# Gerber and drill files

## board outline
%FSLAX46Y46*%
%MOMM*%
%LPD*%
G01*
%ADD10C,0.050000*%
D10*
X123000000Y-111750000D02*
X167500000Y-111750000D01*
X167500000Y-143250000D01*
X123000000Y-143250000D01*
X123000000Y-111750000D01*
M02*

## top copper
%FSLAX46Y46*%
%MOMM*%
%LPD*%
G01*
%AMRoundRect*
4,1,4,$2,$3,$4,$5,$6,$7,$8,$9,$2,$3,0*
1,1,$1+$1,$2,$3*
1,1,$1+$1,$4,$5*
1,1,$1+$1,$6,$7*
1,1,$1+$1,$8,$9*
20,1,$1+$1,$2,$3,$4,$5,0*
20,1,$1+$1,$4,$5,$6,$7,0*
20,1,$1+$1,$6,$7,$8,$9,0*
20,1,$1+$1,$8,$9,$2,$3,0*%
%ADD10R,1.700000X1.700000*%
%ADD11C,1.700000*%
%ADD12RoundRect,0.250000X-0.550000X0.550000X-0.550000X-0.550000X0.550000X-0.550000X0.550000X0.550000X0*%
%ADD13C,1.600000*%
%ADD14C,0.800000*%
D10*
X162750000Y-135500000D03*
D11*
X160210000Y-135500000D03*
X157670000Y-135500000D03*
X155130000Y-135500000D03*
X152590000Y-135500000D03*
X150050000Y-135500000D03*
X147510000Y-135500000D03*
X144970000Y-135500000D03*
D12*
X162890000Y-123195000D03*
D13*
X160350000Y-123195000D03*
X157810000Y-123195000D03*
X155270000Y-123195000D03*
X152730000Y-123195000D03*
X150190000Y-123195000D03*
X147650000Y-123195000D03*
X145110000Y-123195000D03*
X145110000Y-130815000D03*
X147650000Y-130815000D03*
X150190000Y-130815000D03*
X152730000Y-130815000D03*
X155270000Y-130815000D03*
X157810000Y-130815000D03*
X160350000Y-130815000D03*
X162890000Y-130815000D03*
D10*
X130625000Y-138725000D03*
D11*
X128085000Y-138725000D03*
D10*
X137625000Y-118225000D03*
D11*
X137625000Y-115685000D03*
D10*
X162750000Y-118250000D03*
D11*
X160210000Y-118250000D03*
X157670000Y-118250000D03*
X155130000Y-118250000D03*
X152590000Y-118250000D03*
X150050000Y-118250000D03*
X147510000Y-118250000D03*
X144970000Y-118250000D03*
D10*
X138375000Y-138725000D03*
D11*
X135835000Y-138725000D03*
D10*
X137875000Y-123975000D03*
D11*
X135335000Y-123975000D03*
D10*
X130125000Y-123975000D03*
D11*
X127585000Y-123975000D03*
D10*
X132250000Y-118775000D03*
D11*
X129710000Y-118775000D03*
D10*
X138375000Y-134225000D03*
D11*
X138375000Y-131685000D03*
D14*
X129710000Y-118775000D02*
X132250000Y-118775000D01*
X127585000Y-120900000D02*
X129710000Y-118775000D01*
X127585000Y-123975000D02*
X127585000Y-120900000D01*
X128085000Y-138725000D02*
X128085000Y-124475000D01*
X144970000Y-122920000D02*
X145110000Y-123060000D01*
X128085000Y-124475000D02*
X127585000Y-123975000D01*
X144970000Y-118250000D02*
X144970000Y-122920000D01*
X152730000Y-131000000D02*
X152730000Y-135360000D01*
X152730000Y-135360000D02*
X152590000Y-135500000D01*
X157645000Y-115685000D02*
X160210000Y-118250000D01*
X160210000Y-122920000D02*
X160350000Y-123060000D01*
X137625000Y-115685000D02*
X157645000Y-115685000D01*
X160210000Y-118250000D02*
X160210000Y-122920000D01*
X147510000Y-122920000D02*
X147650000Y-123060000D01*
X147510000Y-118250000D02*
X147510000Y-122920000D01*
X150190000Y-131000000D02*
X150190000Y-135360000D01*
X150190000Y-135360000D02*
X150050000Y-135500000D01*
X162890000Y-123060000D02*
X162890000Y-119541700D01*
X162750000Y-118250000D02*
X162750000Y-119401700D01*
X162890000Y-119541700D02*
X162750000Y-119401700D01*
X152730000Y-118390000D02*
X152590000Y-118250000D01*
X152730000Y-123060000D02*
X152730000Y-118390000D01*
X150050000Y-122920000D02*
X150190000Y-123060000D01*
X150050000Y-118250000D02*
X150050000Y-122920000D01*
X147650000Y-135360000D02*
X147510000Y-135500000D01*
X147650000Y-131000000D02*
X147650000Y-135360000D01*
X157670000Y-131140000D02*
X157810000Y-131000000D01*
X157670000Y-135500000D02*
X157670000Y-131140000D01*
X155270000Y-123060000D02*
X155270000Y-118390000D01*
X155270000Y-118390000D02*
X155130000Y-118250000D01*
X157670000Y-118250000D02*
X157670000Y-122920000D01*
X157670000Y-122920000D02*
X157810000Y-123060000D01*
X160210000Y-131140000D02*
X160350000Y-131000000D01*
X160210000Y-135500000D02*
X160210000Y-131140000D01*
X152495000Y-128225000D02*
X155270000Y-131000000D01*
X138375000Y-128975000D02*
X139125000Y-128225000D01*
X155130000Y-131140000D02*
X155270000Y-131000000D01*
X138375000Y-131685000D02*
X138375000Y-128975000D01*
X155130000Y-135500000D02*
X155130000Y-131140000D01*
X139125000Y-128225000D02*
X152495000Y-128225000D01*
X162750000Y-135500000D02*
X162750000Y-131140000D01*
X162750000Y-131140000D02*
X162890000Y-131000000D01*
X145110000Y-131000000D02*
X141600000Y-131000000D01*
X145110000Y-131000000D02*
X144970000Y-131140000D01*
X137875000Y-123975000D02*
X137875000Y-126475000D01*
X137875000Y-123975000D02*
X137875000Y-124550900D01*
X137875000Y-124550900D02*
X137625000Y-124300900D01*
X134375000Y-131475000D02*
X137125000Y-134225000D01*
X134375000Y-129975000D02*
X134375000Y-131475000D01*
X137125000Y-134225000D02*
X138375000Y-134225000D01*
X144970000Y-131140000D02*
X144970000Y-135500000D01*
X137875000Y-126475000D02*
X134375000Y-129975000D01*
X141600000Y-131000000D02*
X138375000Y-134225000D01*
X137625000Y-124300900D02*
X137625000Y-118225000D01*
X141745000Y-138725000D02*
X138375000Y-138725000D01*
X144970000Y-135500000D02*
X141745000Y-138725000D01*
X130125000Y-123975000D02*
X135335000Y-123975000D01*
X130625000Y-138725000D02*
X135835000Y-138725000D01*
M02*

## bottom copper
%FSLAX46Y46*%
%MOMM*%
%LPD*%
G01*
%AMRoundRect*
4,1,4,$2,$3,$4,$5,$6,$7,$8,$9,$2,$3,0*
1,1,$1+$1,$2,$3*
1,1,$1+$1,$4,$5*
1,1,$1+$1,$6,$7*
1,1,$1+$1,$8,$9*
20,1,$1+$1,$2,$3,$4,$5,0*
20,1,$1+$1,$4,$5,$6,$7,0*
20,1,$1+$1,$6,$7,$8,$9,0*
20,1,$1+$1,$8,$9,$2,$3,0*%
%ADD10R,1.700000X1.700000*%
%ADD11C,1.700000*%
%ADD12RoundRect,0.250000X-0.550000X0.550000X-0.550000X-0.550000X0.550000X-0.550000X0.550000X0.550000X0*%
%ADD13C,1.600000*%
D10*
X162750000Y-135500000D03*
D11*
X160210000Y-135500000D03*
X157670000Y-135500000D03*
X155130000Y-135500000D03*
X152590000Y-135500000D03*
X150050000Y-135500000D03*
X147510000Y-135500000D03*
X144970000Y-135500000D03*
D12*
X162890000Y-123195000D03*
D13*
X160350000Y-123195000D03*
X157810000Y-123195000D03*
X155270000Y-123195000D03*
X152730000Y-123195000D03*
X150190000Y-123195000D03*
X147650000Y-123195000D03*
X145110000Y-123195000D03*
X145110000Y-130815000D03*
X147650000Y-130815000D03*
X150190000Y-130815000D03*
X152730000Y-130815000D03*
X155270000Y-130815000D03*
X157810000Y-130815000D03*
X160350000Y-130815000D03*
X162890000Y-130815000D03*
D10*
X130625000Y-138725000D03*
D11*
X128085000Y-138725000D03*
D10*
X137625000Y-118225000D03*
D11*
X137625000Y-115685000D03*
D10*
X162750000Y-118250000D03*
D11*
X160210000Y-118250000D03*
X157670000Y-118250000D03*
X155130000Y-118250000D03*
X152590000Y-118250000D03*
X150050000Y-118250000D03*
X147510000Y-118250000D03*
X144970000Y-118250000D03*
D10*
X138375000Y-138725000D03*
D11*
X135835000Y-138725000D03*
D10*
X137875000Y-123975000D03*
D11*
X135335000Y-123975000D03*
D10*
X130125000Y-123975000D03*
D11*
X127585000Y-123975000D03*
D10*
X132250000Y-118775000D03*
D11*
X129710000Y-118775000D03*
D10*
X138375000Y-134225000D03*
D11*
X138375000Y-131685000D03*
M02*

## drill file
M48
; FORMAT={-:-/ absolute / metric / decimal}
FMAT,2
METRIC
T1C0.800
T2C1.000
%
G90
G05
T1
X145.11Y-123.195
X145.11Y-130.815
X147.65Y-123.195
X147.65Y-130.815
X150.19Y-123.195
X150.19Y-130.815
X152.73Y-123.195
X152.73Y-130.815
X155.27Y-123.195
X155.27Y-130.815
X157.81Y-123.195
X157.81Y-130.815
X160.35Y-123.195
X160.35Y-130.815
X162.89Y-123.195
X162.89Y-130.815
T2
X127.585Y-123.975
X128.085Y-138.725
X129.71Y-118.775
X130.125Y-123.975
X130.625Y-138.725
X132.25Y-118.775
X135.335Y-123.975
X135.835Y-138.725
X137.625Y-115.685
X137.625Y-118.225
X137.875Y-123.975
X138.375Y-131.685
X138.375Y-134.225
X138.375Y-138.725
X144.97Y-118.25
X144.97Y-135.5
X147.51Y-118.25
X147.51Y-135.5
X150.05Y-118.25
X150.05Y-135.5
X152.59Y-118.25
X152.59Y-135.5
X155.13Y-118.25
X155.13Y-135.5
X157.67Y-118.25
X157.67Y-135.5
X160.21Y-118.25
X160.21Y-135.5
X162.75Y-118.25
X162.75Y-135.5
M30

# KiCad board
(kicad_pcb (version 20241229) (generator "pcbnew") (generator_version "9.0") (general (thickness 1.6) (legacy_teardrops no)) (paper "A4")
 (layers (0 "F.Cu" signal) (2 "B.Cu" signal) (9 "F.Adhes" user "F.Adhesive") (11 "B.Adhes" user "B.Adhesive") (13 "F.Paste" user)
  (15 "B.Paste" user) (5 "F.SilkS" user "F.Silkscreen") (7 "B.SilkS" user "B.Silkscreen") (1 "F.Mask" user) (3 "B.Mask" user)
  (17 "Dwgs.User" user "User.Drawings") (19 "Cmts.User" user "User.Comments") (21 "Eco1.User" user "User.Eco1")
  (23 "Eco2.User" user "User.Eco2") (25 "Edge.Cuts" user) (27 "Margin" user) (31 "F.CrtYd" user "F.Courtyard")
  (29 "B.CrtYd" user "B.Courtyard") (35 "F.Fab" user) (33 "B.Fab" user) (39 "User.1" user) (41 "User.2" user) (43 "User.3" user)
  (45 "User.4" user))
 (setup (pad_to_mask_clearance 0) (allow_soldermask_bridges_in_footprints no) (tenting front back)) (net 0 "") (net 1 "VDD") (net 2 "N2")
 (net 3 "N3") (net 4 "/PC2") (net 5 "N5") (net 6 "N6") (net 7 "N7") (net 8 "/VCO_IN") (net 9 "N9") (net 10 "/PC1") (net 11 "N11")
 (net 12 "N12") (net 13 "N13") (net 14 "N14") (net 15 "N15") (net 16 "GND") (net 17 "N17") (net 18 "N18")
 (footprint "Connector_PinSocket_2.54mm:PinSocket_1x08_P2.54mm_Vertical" (layer "F.Cu") (at 162.75 135.5 -90)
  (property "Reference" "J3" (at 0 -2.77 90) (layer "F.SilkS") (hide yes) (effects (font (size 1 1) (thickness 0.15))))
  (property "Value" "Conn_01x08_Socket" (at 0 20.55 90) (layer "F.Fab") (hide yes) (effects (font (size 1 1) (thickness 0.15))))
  (pad "1" thru_hole rect (at 0 0 270) (size 1.7 1.7) (drill 1) (layers "*.Cu" "*.Mask") (remove_unused_layers no) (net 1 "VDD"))
  (pad "2" thru_hole circle (at 0 2.54 270) (size 1.7 1.7) (drill 1) (layers "*.Cu" "*.Mask") (remove_unused_layers no) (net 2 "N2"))
  (pad "3" thru_hole circle (at 0 5.08 270) (size 1.7 1.7) (drill 1) (layers "*.Cu" "*.Mask") (remove_unused_layers no) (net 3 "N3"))
  (pad "4" thru_hole circle (at 0 7.62 270) (size 1.7 1.7) (drill 1) (layers "*.Cu" "*.Mask") (remove_unused_layers no) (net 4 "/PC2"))
  (pad "5" thru_hole circle (at 0 10.16 270) (size 1.7 1.7) (drill 1) (layers "*.Cu" "*.Mask") (remove_unused_layers no) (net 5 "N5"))
  (pad "6" thru_hole circle (at 0 12.7 270) (size 1.7 1.7) (drill 1) (layers "*.Cu" "*.Mask") (remove_unused_layers no) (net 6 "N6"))
  (pad "7" thru_hole circle (at 0 15.24 270) (size 1.7 1.7) (drill 1) (layers "*.Cu" "*.Mask") (remove_unused_layers no) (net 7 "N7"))
  (pad "8" thru_hole circle (at 0 17.78 270) (size 1.7 1.7) (drill 1) (layers "*.Cu" "*.Mask") (remove_unused_layers no) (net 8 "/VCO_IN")))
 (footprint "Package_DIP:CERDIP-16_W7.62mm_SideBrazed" (layer "F.Cu") (at 162.89 123.195 -90)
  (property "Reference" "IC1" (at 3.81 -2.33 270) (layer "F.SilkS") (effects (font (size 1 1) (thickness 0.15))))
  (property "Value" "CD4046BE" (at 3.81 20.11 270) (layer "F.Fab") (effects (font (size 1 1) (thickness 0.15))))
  (pad "1" thru_hole roundrect (at 0 0 270) (size 1.6 1.6) (drill 0.8) (layers "*.Cu" "*.Mask") (remove_unused_layers no)
   (roundrect_rratio 0.15625) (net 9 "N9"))
  (pad "2" thru_hole circle (at 0 2.54 270) (size 1.6 1.6) (drill 0.8) (layers "*.Cu" "*.Mask") (remove_unused_layers no) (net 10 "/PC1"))
  (pad "3" thru_hole circle (at 0 5.08 270) (size 1.6 1.6) (drill 0.8) (layers "*.Cu" "*.Mask") (remove_unused_layers no) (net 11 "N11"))
  (pad "4" thru_hole circle (at 0 7.62 270) (size 1.6 1.6) (drill 0.8) (layers "*.Cu" "*.Mask") (remove_unused_layers no) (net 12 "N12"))
  (pad "5" thru_hole circle (at 0 10.16 270) (size 1.6 1.6) (drill 0.8) (layers "*.Cu" "*.Mask") (remove_unused_layers no) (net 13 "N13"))
  (pad "6" thru_hole circle (at 0 12.7 270) (size 1.6 1.6) (drill 0.8) (layers "*.Cu" "*.Mask") (remove_unused_layers no) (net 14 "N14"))
  (pad "7" thru_hole circle (at 0 15.24 270) (size 1.6 1.6) (drill 0.8) (layers "*.Cu" "*.Mask") (remove_unused_layers no) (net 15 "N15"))
  (pad "8" thru_hole circle (at 0 17.78 270) (size 1.6 1.6) (drill 0.8) (layers "*.Cu" "*.Mask") (remove_unused_layers no) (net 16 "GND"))
  (pad "9" thru_hole circle (at 7.62 17.78 270) (size 1.6 1.6) (drill 0.8) (layers "*.Cu" "*.Mask") (remove_unused_layers no)
   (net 8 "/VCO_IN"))
  (pad "10" thru_hole circle (at 7.62 15.24 270) (size 1.6 1.6) (drill 0.8) (layers "*.Cu" "*.Mask") (remove_unused_layers no) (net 7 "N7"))
  (pad "11" thru_hole circle (at 7.62 12.7 270) (size 1.6 1.6) (drill 0.8) (layers "*.Cu" "*.Mask") (remove_unused_layers no) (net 6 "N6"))
  (pad "12" thru_hole circle (at 7.62 10.16 270) (size 1.6 1.6) (drill 0.8) (layers "*.Cu" "*.Mask") (remove_unused_layers no) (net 5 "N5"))
  (pad "13" thru_hole circle (at 7.62 7.62 270) (size 1.6 1.6) (drill 0.8) (layers "*.Cu" "*.Mask") (remove_unused_layers no) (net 4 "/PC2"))
  (pad "14" thru_hole circle (at 7.62 5.08 270) (size 1.6 1.6) (drill 0.8) (layers "*.Cu" "*.Mask") (remove_unused_layers no) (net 3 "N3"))
  (pad "15" thru_hole circle (at 7.62 2.54 270) (size 1.6 1.6) (drill 0.8) (layers "*.Cu" "*.Mask") (remove_unused_layers no) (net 2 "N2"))
  (pad "16" thru_hole circle (at 7.62 0 270) (size 1.6 1.6) (drill 0.8) (layers "*.Cu" "*.Mask") (remove_unused_layers no) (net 1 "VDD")))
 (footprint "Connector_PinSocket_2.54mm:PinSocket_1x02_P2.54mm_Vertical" (layer "F.Cu") (at 130.625 138.725 -90)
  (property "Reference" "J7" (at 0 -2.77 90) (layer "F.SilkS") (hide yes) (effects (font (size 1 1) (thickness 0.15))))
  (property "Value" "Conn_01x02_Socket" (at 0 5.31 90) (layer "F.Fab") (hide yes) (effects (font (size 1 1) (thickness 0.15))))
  (pad "1" thru_hole rect (at 0 0 270) (size 1.7 1.7) (drill 1) (layers "*.Cu" "*.Mask") (remove_unused_layers no) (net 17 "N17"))
  (pad "2" thru_hole circle (at 0 2.54 270) (size 1.7 1.7) (drill 1) (layers "*.Cu" "*.Mask") (remove_unused_layers no) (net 16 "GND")))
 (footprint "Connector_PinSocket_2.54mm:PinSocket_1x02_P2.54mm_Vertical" (layer "F.Cu") (at 137.625 118.225 180)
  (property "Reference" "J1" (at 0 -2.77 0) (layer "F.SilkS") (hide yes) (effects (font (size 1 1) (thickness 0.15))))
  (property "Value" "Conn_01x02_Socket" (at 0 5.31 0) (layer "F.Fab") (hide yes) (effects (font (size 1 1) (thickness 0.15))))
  (pad "1" thru_hole rect (at 0 0 180) (size 1.7 1.7) (drill 1) (layers "*.Cu" "*.Mask") (remove_unused_layers no) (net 8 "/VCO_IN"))
  (pad "2" thru_hole circle (at 0 2.54 180) (size 1.7 1.7) (drill 1) (layers "*.Cu" "*.Mask") (remove_unused_layers no) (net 10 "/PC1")))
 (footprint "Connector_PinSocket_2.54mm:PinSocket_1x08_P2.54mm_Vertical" (layer "F.Cu") (at 162.75 118.25 -90)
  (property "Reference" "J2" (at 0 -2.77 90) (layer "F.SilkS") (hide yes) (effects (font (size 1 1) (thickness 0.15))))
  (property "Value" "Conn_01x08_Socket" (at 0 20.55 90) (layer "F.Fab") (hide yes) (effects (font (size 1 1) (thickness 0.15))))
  (pad "1" thru_hole rect (at 0 0 270) (size 1.7 1.7) (drill 1) (layers "*.Cu" "*.Mask") (remove_unused_layers no) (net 9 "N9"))
  (pad "2" thru_hole circle (at 0 2.54 270) (size 1.7 1.7) (drill 1) (layers "*.Cu" "*.Mask") (remove_unused_layers no) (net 10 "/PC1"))
  (pad "3" thru_hole circle (at 0 5.08 270) (size 1.7 1.7) (drill 1) (layers "*.Cu" "*.Mask") (remove_unused_layers no) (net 11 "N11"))
  (pad "4" thru_hole circle (at 0 7.62 270) (size 1.7 1.7) (drill 1) (layers "*.Cu" "*.Mask") (remove_unused_layers no) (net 12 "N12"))
  (pad "5" thru_hole circle (at 0 10.16 270) (size 1.7 1.7) (drill 1) (layers "*.Cu" "*.Mask") (remove_unused_layers no) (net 13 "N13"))
  (pad "6" thru_hole circle (at 0 12.7 270) (size 1.7 1.7) (drill 1) (layers "*.Cu" "*.Mask") (remove_unused_layers no) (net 14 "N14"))
  (pad "7" thru_hole circle (at 0 15.24 270) (size 1.7 1.7) (drill 1) (layers "*.Cu" "*.Mask") (remove_unused_layers no) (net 15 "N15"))
  (pad "8" thru_hole circle (at 0 17.78 270) (size 1.7 1.7) (drill 1) (layers "*.Cu" "*.Mask") (remove_unused_layers no) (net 16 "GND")))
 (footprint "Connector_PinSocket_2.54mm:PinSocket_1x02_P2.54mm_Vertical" (layer "F.Cu") (at 138.375 138.725 -90)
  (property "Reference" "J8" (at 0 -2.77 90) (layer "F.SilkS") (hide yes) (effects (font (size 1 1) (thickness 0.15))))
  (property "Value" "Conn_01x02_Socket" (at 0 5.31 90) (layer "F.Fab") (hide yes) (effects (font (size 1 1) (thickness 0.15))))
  (pad "1" thru_hole rect (at 0 0 270) (size 1.7 1.7) (drill 1) (layers "*.Cu" "*.Mask") (remove_unused_layers no) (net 8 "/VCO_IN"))
  (pad "2" thru_hole circle (at 0 2.54 270) (size 1.7 1.7) (drill 1) (layers "*.Cu" "*.Mask") (remove_unused_layers no) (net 17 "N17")))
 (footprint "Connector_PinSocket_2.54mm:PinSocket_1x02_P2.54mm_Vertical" (layer "F.Cu") (at 137.875 123.975 -90)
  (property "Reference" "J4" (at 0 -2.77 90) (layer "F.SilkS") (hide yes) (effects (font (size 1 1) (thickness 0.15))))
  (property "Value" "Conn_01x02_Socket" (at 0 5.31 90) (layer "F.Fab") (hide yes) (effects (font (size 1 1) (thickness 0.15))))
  (pad "1" thru_hole rect (at 0 0 270) (size 1.7 1.7) (drill 1) (layers "*.Cu" "*.Mask") (remove_unused_layers no) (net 8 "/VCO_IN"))
  (pad "2" thru_hole circle (at 0 2.54 270) (size 1.7 1.7) (drill 1) (layers "*.Cu" "*.Mask") (remove_unused_layers no) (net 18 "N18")))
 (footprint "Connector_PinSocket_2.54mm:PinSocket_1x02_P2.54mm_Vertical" (layer "F.Cu") (at 130.125 123.975 -90)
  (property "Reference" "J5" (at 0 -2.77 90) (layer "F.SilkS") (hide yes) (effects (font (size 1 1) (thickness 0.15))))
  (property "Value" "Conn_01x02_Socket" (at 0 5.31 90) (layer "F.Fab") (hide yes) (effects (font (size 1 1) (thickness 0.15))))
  (pad "1" thru_hole rect (at 0 0 270) (size 1.7 1.7) (drill 1) (layers "*.Cu" "*.Mask") (remove_unused_layers no) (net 18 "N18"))
  (pad "2" thru_hole circle (at 0 2.54 270) (size 1.7 1.7) (drill 1) (layers "*.Cu" "*.Mask") (remove_unused_layers no) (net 16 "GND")))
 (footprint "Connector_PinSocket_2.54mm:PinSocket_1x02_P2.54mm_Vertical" (layer "F.Cu") (at 132.25 118.775 -90)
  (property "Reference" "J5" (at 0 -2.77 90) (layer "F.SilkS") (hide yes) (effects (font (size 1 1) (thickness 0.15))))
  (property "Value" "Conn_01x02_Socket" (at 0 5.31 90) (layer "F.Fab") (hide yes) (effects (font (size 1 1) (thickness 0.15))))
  (pad "1" thru_hole rect (at 0 0 270) (size 1.7 1.7) (drill 1) (layers "*.Cu" "*.Mask") (remove_unused_layers no) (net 16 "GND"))
  (pad "2" thru_hole circle (at 0 2.54 270) (size 1.7 1.7) (drill 1) (layers "*.Cu" "*.Mask") (remove_unused_layers no) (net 16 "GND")))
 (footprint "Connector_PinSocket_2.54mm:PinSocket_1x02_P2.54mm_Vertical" (layer "F.Cu") (at 138.375 134.225 180)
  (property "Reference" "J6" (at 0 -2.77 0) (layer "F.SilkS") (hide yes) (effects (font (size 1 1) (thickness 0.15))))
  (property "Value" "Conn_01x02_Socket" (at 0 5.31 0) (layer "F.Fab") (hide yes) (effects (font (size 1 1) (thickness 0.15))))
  (pad "1" thru_hole rect (at 0 0 180) (size 1.7 1.7) (drill 1) (layers "*.Cu" "*.Mask") (remove_unused_layers no) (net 8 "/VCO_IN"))
  (pad "2" thru_hole circle (at 0 2.54 180) (size 1.7 1.7) (drill 1) (layers "*.Cu" "*.Mask") (remove_unused_layers no) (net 4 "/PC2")))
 (gr_rect (start 123 111.75) (end 167.5 143.25) (stroke (width 0.05) (type default)) (fill no) (layer "Edge.Cuts"))
 (segment (start 129.71 118.775) (end 132.25 118.775) (width 0.8) (layer "F.Cu") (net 16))
 (segment (start 127.585 120.9) (end 129.71 118.775) (width 0.8) (layer "F.Cu") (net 16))
 (segment (start 127.585 123.975) (end 127.585 120.9) (width 0.8) (layer "F.Cu") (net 16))
 (segment (start 128.085 138.725) (end 128.085 124.475) (width 0.8) (layer "F.Cu") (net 16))
 (segment (start 144.97 122.92) (end 145.11 123.06) (width 0.8) (layer "F.Cu") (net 16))
 (segment (start 128.085 124.475) (end 127.585 123.975) (width 0.8) (layer "F.Cu") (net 16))
 (segment (start 144.97 118.25) (end 144.97 122.92) (width 0.8) (layer "F.Cu") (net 16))
 (segment (start 152.73 131) (end 152.73 135.36) (width 0.8) (layer "F.Cu") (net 5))
 (segment (start 152.73 135.36) (end 152.59 135.5) (width 0.8) (layer "F.Cu") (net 5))
 (segment (start 157.645 115.685) (end 160.21 118.25) (width 0.8) (layer "F.Cu") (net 10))
 (segment (start 160.21 122.92) (end 160.35 123.06) (width 0.8) (layer "F.Cu") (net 10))
 (segment (start 137.625 115.685) (end 157.645 115.685) (width 0.8) (layer "F.Cu") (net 10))
 (segment (start 160.21 118.25) (end 160.21 122.92) (width 0.8) (layer "F.Cu") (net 10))
 (segment (start 147.51 122.92) (end 147.65 123.06) (width 0.8) (layer "F.Cu") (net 15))
 (segment (start 147.51 118.25) (end 147.51 122.92) (width 0.8) (layer "F.Cu") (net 15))
 (segment (start 150.19 131) (end 150.19 135.36) (width 0.8) (layer "F.Cu") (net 6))
 (segment (start 150.19 135.36) (end 150.05 135.5) (width 0.8) (layer "F.Cu") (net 6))
 (segment (start 162.89 123.06) (end 162.89 119.5417) (width 0.8) (layer "F.Cu") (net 9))
 (segment (start 162.75 118.25) (end 162.75 119.4017) (width 0.8) (layer "F.Cu") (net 9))
 (segment (start 162.89 119.5417) (end 162.75 119.4017) (width 0.8) (layer "F.Cu") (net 9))
 (segment (start 152.73 118.39) (end 152.59 118.25) (width 0.8) (layer "F.Cu") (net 13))
 (segment (start 152.73 123.06) (end 152.73 118.39) (width 0.8) (layer "F.Cu") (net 13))
 (segment (start 150.05 122.92) (end 150.19 123.06) (width 0.8) (layer "F.Cu") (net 14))
 (segment (start 150.05 118.25) (end 150.05 122.92) (width 0.8) (layer "F.Cu") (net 14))
 (segment (start 147.65 135.36) (end 147.51 135.5) (width 0.8) (layer "F.Cu") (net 7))
 (segment (start 147.65 131) (end 147.65 135.36) (width 0.8) (layer "F.Cu") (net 7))
 (segment (start 157.67 131.14) (end 157.81 131) (width 0.8) (layer "F.Cu") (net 3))
 (segment (start 157.67 135.5) (end 157.67 131.14) (width 0.8) (layer "F.Cu") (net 3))
 (segment (start 155.27 123.06) (end 155.27 118.39) (width 0.8) (layer "F.Cu") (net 12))
 (segment (start 155.27 118.39) (end 155.13 118.25) (width 0.8) (layer "F.Cu") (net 12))
 (segment (start 157.67 118.25) (end 157.67 122.92) (width 0.8) (layer "F.Cu") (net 11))
 (segment (start 157.67 122.92) (end 157.81 123.06) (width 0.8) (layer "F.Cu") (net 11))
 (segment (start 160.21 131.14) (end 160.35 131) (width 0.8) (layer "F.Cu") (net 2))
 (segment (start 160.21 135.5) (end 160.21 131.14) (width 0.8) (layer "F.Cu") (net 2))
 (segment (start 152.495 128.225) (end 155.27 131) (width 0.8) (layer "F.Cu") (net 4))
 (segment (start 138.375 128.975) (end 139.125 128.225) (width 0.8) (layer "F.Cu") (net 4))
 (segment (start 155.13 131.14) (end 155.27 131) (width 0.8) (layer "F.Cu") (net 4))
 (segment (start 138.375 131.685) (end 138.375 128.975) (width 0.8) (layer "F.Cu") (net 4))
 (segment (start 155.13 135.5) (end 155.13 131.14) (width 0.8) (layer "F.Cu") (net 4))
 (segment (start 139.125 128.225) (end 152.495 128.225) (width 0.8) (layer "F.Cu") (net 4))
 (segment (start 162.75 135.5) (end 162.75 131.14) (width 0.8) (layer "F.Cu") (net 1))
 (segment (start 162.75 131.14) (end 162.89 131) (width 0.8) (layer "F.Cu") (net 1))
 (segment (start 145.11 131) (end 141.6 131) (width 0.8) (layer "F.Cu") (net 8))
 (segment (start 145.11 131) (end 144.97 131.14) (width 0.8) (layer "F.Cu") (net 8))
 (segment (start 137.875 123.975) (end 137.875 126.475) (width 0.8) (layer "F.Cu") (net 8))
 (segment (start 137.875 123.975) (end 137.875 124.5509) (width 0.8) (layer "F.Cu") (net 8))
 (segment (start 137.875 124.5509) (end 137.625 124.3009) (width 0.8) (layer "F.Cu") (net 8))
 (segment (start 134.375 131.475) (end 137.125 134.225) (width 0.8) (layer "F.Cu") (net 8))
 (segment (start 134.375 129.975) (end 134.375 131.475) (width 0.8) (layer "F.Cu") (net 8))
 (segment (start 137.125 134.225) (end 138.375 134.225) (width 0.8) (layer "F.Cu") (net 8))
 (segment (start 144.97 131.14) (end 144.97 135.5) (width 0.8) (layer "F.Cu") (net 8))
 (segment (start 137.875 126.475) (end 134.375 129.975) (width 0.8) (layer "F.Cu") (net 8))
 (segment (start 141.6 131) (end 138.375 134.225) (width 0.8) (layer "F.Cu") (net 8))
 (segment (start 137.625 124.3009) (end 137.625 118.225) (width 0.8) (layer "F.Cu") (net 8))
 (segment (start 141.745 138.725) (end 138.375 138.725) (width 0.8) (layer "F.Cu") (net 8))
 (segment (start 144.97 135.5) (end 141.745 138.725) (width 0.8) (layer "F.Cu") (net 8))
 (segment (start 130.125 123.975) (end 135.335 123.975) (width 0.8) (layer "F.Cu") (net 18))
 (segment (start 130.625 138.725) (end 135.835 138.725) (width 0.8) (layer "F.Cu") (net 17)))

